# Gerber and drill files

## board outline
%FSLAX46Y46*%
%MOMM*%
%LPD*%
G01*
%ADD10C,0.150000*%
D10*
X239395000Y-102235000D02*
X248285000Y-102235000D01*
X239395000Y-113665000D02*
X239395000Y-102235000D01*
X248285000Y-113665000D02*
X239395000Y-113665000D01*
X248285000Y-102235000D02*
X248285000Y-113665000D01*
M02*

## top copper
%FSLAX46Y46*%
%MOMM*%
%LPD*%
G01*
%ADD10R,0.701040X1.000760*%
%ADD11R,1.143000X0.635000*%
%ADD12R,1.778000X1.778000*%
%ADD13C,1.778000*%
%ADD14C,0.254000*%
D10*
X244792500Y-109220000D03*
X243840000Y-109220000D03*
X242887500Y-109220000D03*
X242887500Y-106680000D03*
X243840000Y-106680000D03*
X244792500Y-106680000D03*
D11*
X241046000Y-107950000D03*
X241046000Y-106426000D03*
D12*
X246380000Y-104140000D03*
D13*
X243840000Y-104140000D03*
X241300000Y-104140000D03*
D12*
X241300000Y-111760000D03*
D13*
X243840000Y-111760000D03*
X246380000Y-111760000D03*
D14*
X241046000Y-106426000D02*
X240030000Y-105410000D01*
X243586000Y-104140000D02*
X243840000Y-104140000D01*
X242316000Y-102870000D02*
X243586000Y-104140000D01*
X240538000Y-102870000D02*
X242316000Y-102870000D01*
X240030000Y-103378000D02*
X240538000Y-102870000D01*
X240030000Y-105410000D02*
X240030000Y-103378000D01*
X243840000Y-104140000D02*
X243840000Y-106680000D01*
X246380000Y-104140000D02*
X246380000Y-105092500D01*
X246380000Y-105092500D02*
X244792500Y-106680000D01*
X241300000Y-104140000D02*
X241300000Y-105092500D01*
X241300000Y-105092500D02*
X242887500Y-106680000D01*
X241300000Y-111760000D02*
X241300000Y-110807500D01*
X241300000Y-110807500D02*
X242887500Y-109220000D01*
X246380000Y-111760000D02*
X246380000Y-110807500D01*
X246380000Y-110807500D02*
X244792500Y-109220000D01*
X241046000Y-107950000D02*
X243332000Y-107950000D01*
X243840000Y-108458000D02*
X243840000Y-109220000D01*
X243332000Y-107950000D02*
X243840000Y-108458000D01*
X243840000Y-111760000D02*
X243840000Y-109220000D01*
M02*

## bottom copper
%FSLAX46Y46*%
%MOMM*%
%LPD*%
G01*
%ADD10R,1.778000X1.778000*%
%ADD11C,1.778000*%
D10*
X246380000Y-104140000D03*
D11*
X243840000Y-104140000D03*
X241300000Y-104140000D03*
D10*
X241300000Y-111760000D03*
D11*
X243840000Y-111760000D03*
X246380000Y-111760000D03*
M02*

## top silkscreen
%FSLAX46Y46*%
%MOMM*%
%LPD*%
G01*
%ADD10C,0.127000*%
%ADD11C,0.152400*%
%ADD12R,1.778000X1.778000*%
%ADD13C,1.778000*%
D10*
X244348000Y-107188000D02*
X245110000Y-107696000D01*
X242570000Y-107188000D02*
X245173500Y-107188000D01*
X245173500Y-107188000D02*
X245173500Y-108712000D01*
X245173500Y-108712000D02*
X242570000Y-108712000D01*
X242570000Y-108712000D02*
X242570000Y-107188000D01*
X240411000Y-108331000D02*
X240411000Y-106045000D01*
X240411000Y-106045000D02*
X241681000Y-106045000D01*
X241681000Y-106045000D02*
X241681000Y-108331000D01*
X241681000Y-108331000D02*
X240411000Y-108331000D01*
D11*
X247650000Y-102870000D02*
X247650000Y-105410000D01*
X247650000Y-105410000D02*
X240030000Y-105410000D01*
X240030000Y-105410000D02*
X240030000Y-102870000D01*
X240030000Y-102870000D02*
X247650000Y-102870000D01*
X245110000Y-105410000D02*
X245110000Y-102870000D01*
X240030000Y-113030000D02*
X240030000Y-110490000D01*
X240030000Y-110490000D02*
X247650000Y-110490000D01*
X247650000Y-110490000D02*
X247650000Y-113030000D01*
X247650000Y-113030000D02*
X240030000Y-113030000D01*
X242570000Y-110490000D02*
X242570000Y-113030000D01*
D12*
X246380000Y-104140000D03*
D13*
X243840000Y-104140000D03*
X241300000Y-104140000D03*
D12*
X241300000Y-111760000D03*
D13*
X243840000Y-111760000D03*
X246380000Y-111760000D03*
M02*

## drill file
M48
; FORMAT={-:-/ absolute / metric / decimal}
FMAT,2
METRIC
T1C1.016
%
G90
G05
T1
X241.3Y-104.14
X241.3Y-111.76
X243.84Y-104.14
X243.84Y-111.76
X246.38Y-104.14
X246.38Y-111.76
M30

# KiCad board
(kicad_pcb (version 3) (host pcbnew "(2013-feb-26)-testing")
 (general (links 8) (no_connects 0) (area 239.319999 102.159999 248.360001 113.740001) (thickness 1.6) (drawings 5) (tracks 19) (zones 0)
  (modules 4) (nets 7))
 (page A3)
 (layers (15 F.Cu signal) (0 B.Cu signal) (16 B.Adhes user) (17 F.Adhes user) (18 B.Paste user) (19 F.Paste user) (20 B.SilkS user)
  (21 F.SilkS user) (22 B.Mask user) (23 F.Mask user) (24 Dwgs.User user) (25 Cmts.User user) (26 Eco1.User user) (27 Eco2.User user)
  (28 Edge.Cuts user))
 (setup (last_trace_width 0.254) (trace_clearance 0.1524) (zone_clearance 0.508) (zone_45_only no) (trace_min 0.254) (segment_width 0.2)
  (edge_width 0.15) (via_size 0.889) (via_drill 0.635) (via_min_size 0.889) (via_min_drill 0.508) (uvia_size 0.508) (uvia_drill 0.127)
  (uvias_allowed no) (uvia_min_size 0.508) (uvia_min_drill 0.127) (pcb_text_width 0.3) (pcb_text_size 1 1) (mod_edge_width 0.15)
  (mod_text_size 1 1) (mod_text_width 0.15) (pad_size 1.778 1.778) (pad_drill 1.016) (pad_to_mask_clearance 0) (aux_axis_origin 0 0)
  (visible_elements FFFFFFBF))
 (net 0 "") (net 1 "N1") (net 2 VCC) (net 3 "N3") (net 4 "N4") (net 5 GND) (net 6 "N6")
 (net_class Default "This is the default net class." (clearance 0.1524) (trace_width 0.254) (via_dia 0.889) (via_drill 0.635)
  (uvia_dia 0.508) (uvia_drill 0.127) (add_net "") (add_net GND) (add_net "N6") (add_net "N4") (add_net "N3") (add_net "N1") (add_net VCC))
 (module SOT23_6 (layer F.Cu) (at 243.84 107.95 180)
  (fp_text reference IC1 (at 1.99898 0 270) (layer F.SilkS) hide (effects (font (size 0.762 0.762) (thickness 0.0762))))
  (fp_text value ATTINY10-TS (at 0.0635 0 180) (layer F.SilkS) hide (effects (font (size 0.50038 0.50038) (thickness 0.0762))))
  (fp_line (start -0.508 0.762) (end -1.27 0.254) (layer F.SilkS) (width 0.127))
  (fp_line (start 1.27 0.762) (end -1.3335 0.762) (layer F.SilkS) (width 0.127))
  (fp_line (start -1.3335 0.762) (end -1.3335 -0.762) (layer F.SilkS) (width 0.127))
  (fp_line (start -1.3335 -0.762) (end 1.27 -0.762) (layer F.SilkS) (width 0.127))
  (fp_line (start 1.27 -0.762) (end 1.27 0.762) (layer F.SilkS) (width 0.127))
  (pad 6 smd rect (at -0.9525 -1.27 180) (size 0.70104 1.00076) (layers F.Cu F.Paste F.Mask) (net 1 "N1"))
  (pad 5 smd rect (at 0 -1.27 180) (size 0.70104 1.00076) (layers F.Cu F.Paste F.Mask) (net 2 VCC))
  (pad 4 smd rect (at 0.9525 -1.27 180) (size 0.70104 1.00076) (layers F.Cu F.Paste F.Mask) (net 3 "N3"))
  (pad 3 smd rect (at 0.9525 1.27 180) (size 0.70104 1.00076) (layers F.Cu F.Paste F.Mask) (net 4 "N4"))
  (pad 2 smd rect (at 0 1.27 180) (size 0.70104 1.00076) (layers F.Cu F.Paste F.Mask) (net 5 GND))
  (pad 1 smd rect (at -0.9525 1.27 180) (size 0.70104 1.00076) (layers F.Cu F.Paste F.Mask) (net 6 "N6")))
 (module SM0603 (layer F.Cu) (at 241.046 107.188 90)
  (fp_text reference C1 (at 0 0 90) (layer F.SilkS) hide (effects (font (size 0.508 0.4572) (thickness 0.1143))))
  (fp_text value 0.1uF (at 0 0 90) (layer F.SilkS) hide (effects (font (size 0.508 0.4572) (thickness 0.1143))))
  (fp_line (start -1.143 -0.635) (end 1.143 -0.635) (layer F.SilkS) (width 0.127))
  (fp_line (start 1.143 -0.635) (end 1.143 0.635) (layer F.SilkS) (width 0.127))
  (fp_line (start 1.143 0.635) (end -1.143 0.635) (layer F.SilkS) (width 0.127))
  (fp_line (start -1.143 0.635) (end -1.143 -0.635) (layer F.SilkS) (width 0.127))
  (pad 1 smd rect (at -0.762 0 90) (size 0.635 1.143) (layers F.Cu F.Paste F.Mask) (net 2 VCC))
  (pad 2 smd rect (at 0.762 0 90) (size 0.635 1.143) (layers F.Cu F.Paste F.Mask) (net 5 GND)))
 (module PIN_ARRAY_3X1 (layer F.Cu) (at 243.84 104.14 180)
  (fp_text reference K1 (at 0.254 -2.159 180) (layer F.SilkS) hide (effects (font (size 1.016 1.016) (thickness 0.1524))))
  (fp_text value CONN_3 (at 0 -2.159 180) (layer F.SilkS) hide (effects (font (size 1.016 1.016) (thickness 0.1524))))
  (fp_line (start -3.81 1.27) (end -3.81 -1.27) (layer F.SilkS) (width 0.1524))
  (fp_line (start -3.81 -1.27) (end 3.81 -1.27) (layer F.SilkS) (width 0.1524))
  (fp_line (start 3.81 -1.27) (end 3.81 1.27) (layer F.SilkS) (width 0.1524))
  (fp_line (start 3.81 1.27) (end -3.81 1.27) (layer F.SilkS) (width 0.1524))
  (fp_line (start -1.27 -1.27) (end -1.27 1.27) (layer F.SilkS) (width 0.1524))
  (pad 1 thru_hole rect (at -2.54 0 180) (size 1.778 1.778) (drill 1.016) (layers *.Cu *.Mask F.SilkS) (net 6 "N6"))
  (pad 2 thru_hole circle (at 0 0 180) (size 1.778 1.778) (drill 1.016) (layers *.Cu *.Mask F.SilkS) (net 5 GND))
  (pad 3 thru_hole circle (at 2.54 0 180) (size 1.778 1.778) (drill 1.016) (layers *.Cu *.Mask F.SilkS) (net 4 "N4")))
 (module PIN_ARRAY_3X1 (layer F.Cu) (at 243.84 111.76)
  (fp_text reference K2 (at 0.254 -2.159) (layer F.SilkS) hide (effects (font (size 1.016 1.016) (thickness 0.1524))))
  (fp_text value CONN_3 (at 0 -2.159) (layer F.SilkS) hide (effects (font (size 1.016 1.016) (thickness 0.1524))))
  (fp_line (start -3.81 1.27) (end -3.81 -1.27) (layer F.SilkS) (width 0.1524))
  (fp_line (start -3.81 -1.27) (end 3.81 -1.27) (layer F.SilkS) (width 0.1524))
  (fp_line (start 3.81 -1.27) (end 3.81 1.27) (layer F.SilkS) (width 0.1524))
  (fp_line (start 3.81 1.27) (end -3.81 1.27) (layer F.SilkS) (width 0.1524))
  (fp_line (start -1.27 -1.27) (end -1.27 1.27) (layer F.SilkS) (width 0.1524))
  (pad 1 thru_hole rect (at -2.54 0) (size 1.778 1.778) (drill 1.016) (layers *.Cu *.Mask F.SilkS) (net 3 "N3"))
  (pad 2 thru_hole circle (at 0 0) (size 1.778 1.778) (drill 1.016) (layers *.Cu *.Mask F.SilkS) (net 2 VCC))
  (pad 3 thru_hole circle (at 2.54 0) (size 1.778 1.778) (drill 1.016) (layers *.Cu *.Mask F.SilkS) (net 1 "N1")))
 (gr_line (start 239.395 102.235) (end 248.285 102.235) (angle 90) (layer Edge.Cuts) (width 0.15))
 (gr_line (start 239.395 113.665) (end 239.395 102.235) (angle 90) (layer Edge.Cuts) (width 0.15))
 (gr_line (start 248.285 113.665) (end 239.395 113.665) (angle 90) (layer Edge.Cuts) (width 0.15))
 (gr_line (start 248.285 102.235) (end 248.285 113.665) (angle 90) (layer Edge.Cuts) (width 0.15))
 (segment (start 241.046 106.426) (end 240.03 105.41) (width 0.254) (layer F.Cu) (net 5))
 (segment (start 243.586 104.14) (end 243.84 104.14) (width 0.254) (layer F.Cu) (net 5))
 (segment (start 242.316 102.87) (end 243.586 104.14) (width 0.254) (layer F.Cu) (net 5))
 (segment (start 240.538 102.87) (end 242.316 102.87) (width 0.254) (layer F.Cu) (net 5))
 (segment (start 240.03 103.378) (end 240.538 102.87) (width 0.254) (layer F.Cu) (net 5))
 (segment (start 240.03 105.41) (end 240.03 103.378) (width 0.254) (layer F.Cu) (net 5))
 (segment (start 243.84 104.14) (end 243.84 106.68) (width 0.254) (layer F.Cu) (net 5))
 (segment (start 246.38 104.14) (end 246.38 105.0925) (width 0.254) (layer F.Cu) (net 6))
 (segment (start 246.38 105.0925) (end 244.7925 106.68) (width 0.254) (layer F.Cu) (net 6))
 (segment (start 241.3 104.14) (end 241.3 105.0925) (width 0.254) (layer F.Cu) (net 4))
 (segment (start 241.3 105.0925) (end 242.8875 106.68) (width 0.254) (layer F.Cu) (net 4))
 (segment (start 241.3 111.76) (end 241.3 110.8075) (width 0.254) (layer F.Cu) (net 3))
 (segment (start 241.3 110.8075) (end 242.8875 109.22) (width 0.254) (layer F.Cu) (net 3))
 (segment (start 246.38 111.76) (end 246.38 110.8075) (width 0.254) (layer F.Cu) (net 1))
 (segment (start 246.38 110.8075) (end 244.7925 109.22) (width 0.254) (layer F.Cu) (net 1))
 (segment (start 241.046 107.95) (end 243.332 107.95) (width 0.254) (layer F.Cu) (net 2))
 (segment (start 243.84 108.458) (end 243.84 109.22) (width 0.254) (layer F.Cu) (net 2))
 (segment (start 243.332 107.95) (end 243.84 108.458) (width 0.254) (layer F.Cu) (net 2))
 (segment (start 243.84 111.76) (end 243.84 109.22) (width 0.254) (layer F.Cu) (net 2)))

